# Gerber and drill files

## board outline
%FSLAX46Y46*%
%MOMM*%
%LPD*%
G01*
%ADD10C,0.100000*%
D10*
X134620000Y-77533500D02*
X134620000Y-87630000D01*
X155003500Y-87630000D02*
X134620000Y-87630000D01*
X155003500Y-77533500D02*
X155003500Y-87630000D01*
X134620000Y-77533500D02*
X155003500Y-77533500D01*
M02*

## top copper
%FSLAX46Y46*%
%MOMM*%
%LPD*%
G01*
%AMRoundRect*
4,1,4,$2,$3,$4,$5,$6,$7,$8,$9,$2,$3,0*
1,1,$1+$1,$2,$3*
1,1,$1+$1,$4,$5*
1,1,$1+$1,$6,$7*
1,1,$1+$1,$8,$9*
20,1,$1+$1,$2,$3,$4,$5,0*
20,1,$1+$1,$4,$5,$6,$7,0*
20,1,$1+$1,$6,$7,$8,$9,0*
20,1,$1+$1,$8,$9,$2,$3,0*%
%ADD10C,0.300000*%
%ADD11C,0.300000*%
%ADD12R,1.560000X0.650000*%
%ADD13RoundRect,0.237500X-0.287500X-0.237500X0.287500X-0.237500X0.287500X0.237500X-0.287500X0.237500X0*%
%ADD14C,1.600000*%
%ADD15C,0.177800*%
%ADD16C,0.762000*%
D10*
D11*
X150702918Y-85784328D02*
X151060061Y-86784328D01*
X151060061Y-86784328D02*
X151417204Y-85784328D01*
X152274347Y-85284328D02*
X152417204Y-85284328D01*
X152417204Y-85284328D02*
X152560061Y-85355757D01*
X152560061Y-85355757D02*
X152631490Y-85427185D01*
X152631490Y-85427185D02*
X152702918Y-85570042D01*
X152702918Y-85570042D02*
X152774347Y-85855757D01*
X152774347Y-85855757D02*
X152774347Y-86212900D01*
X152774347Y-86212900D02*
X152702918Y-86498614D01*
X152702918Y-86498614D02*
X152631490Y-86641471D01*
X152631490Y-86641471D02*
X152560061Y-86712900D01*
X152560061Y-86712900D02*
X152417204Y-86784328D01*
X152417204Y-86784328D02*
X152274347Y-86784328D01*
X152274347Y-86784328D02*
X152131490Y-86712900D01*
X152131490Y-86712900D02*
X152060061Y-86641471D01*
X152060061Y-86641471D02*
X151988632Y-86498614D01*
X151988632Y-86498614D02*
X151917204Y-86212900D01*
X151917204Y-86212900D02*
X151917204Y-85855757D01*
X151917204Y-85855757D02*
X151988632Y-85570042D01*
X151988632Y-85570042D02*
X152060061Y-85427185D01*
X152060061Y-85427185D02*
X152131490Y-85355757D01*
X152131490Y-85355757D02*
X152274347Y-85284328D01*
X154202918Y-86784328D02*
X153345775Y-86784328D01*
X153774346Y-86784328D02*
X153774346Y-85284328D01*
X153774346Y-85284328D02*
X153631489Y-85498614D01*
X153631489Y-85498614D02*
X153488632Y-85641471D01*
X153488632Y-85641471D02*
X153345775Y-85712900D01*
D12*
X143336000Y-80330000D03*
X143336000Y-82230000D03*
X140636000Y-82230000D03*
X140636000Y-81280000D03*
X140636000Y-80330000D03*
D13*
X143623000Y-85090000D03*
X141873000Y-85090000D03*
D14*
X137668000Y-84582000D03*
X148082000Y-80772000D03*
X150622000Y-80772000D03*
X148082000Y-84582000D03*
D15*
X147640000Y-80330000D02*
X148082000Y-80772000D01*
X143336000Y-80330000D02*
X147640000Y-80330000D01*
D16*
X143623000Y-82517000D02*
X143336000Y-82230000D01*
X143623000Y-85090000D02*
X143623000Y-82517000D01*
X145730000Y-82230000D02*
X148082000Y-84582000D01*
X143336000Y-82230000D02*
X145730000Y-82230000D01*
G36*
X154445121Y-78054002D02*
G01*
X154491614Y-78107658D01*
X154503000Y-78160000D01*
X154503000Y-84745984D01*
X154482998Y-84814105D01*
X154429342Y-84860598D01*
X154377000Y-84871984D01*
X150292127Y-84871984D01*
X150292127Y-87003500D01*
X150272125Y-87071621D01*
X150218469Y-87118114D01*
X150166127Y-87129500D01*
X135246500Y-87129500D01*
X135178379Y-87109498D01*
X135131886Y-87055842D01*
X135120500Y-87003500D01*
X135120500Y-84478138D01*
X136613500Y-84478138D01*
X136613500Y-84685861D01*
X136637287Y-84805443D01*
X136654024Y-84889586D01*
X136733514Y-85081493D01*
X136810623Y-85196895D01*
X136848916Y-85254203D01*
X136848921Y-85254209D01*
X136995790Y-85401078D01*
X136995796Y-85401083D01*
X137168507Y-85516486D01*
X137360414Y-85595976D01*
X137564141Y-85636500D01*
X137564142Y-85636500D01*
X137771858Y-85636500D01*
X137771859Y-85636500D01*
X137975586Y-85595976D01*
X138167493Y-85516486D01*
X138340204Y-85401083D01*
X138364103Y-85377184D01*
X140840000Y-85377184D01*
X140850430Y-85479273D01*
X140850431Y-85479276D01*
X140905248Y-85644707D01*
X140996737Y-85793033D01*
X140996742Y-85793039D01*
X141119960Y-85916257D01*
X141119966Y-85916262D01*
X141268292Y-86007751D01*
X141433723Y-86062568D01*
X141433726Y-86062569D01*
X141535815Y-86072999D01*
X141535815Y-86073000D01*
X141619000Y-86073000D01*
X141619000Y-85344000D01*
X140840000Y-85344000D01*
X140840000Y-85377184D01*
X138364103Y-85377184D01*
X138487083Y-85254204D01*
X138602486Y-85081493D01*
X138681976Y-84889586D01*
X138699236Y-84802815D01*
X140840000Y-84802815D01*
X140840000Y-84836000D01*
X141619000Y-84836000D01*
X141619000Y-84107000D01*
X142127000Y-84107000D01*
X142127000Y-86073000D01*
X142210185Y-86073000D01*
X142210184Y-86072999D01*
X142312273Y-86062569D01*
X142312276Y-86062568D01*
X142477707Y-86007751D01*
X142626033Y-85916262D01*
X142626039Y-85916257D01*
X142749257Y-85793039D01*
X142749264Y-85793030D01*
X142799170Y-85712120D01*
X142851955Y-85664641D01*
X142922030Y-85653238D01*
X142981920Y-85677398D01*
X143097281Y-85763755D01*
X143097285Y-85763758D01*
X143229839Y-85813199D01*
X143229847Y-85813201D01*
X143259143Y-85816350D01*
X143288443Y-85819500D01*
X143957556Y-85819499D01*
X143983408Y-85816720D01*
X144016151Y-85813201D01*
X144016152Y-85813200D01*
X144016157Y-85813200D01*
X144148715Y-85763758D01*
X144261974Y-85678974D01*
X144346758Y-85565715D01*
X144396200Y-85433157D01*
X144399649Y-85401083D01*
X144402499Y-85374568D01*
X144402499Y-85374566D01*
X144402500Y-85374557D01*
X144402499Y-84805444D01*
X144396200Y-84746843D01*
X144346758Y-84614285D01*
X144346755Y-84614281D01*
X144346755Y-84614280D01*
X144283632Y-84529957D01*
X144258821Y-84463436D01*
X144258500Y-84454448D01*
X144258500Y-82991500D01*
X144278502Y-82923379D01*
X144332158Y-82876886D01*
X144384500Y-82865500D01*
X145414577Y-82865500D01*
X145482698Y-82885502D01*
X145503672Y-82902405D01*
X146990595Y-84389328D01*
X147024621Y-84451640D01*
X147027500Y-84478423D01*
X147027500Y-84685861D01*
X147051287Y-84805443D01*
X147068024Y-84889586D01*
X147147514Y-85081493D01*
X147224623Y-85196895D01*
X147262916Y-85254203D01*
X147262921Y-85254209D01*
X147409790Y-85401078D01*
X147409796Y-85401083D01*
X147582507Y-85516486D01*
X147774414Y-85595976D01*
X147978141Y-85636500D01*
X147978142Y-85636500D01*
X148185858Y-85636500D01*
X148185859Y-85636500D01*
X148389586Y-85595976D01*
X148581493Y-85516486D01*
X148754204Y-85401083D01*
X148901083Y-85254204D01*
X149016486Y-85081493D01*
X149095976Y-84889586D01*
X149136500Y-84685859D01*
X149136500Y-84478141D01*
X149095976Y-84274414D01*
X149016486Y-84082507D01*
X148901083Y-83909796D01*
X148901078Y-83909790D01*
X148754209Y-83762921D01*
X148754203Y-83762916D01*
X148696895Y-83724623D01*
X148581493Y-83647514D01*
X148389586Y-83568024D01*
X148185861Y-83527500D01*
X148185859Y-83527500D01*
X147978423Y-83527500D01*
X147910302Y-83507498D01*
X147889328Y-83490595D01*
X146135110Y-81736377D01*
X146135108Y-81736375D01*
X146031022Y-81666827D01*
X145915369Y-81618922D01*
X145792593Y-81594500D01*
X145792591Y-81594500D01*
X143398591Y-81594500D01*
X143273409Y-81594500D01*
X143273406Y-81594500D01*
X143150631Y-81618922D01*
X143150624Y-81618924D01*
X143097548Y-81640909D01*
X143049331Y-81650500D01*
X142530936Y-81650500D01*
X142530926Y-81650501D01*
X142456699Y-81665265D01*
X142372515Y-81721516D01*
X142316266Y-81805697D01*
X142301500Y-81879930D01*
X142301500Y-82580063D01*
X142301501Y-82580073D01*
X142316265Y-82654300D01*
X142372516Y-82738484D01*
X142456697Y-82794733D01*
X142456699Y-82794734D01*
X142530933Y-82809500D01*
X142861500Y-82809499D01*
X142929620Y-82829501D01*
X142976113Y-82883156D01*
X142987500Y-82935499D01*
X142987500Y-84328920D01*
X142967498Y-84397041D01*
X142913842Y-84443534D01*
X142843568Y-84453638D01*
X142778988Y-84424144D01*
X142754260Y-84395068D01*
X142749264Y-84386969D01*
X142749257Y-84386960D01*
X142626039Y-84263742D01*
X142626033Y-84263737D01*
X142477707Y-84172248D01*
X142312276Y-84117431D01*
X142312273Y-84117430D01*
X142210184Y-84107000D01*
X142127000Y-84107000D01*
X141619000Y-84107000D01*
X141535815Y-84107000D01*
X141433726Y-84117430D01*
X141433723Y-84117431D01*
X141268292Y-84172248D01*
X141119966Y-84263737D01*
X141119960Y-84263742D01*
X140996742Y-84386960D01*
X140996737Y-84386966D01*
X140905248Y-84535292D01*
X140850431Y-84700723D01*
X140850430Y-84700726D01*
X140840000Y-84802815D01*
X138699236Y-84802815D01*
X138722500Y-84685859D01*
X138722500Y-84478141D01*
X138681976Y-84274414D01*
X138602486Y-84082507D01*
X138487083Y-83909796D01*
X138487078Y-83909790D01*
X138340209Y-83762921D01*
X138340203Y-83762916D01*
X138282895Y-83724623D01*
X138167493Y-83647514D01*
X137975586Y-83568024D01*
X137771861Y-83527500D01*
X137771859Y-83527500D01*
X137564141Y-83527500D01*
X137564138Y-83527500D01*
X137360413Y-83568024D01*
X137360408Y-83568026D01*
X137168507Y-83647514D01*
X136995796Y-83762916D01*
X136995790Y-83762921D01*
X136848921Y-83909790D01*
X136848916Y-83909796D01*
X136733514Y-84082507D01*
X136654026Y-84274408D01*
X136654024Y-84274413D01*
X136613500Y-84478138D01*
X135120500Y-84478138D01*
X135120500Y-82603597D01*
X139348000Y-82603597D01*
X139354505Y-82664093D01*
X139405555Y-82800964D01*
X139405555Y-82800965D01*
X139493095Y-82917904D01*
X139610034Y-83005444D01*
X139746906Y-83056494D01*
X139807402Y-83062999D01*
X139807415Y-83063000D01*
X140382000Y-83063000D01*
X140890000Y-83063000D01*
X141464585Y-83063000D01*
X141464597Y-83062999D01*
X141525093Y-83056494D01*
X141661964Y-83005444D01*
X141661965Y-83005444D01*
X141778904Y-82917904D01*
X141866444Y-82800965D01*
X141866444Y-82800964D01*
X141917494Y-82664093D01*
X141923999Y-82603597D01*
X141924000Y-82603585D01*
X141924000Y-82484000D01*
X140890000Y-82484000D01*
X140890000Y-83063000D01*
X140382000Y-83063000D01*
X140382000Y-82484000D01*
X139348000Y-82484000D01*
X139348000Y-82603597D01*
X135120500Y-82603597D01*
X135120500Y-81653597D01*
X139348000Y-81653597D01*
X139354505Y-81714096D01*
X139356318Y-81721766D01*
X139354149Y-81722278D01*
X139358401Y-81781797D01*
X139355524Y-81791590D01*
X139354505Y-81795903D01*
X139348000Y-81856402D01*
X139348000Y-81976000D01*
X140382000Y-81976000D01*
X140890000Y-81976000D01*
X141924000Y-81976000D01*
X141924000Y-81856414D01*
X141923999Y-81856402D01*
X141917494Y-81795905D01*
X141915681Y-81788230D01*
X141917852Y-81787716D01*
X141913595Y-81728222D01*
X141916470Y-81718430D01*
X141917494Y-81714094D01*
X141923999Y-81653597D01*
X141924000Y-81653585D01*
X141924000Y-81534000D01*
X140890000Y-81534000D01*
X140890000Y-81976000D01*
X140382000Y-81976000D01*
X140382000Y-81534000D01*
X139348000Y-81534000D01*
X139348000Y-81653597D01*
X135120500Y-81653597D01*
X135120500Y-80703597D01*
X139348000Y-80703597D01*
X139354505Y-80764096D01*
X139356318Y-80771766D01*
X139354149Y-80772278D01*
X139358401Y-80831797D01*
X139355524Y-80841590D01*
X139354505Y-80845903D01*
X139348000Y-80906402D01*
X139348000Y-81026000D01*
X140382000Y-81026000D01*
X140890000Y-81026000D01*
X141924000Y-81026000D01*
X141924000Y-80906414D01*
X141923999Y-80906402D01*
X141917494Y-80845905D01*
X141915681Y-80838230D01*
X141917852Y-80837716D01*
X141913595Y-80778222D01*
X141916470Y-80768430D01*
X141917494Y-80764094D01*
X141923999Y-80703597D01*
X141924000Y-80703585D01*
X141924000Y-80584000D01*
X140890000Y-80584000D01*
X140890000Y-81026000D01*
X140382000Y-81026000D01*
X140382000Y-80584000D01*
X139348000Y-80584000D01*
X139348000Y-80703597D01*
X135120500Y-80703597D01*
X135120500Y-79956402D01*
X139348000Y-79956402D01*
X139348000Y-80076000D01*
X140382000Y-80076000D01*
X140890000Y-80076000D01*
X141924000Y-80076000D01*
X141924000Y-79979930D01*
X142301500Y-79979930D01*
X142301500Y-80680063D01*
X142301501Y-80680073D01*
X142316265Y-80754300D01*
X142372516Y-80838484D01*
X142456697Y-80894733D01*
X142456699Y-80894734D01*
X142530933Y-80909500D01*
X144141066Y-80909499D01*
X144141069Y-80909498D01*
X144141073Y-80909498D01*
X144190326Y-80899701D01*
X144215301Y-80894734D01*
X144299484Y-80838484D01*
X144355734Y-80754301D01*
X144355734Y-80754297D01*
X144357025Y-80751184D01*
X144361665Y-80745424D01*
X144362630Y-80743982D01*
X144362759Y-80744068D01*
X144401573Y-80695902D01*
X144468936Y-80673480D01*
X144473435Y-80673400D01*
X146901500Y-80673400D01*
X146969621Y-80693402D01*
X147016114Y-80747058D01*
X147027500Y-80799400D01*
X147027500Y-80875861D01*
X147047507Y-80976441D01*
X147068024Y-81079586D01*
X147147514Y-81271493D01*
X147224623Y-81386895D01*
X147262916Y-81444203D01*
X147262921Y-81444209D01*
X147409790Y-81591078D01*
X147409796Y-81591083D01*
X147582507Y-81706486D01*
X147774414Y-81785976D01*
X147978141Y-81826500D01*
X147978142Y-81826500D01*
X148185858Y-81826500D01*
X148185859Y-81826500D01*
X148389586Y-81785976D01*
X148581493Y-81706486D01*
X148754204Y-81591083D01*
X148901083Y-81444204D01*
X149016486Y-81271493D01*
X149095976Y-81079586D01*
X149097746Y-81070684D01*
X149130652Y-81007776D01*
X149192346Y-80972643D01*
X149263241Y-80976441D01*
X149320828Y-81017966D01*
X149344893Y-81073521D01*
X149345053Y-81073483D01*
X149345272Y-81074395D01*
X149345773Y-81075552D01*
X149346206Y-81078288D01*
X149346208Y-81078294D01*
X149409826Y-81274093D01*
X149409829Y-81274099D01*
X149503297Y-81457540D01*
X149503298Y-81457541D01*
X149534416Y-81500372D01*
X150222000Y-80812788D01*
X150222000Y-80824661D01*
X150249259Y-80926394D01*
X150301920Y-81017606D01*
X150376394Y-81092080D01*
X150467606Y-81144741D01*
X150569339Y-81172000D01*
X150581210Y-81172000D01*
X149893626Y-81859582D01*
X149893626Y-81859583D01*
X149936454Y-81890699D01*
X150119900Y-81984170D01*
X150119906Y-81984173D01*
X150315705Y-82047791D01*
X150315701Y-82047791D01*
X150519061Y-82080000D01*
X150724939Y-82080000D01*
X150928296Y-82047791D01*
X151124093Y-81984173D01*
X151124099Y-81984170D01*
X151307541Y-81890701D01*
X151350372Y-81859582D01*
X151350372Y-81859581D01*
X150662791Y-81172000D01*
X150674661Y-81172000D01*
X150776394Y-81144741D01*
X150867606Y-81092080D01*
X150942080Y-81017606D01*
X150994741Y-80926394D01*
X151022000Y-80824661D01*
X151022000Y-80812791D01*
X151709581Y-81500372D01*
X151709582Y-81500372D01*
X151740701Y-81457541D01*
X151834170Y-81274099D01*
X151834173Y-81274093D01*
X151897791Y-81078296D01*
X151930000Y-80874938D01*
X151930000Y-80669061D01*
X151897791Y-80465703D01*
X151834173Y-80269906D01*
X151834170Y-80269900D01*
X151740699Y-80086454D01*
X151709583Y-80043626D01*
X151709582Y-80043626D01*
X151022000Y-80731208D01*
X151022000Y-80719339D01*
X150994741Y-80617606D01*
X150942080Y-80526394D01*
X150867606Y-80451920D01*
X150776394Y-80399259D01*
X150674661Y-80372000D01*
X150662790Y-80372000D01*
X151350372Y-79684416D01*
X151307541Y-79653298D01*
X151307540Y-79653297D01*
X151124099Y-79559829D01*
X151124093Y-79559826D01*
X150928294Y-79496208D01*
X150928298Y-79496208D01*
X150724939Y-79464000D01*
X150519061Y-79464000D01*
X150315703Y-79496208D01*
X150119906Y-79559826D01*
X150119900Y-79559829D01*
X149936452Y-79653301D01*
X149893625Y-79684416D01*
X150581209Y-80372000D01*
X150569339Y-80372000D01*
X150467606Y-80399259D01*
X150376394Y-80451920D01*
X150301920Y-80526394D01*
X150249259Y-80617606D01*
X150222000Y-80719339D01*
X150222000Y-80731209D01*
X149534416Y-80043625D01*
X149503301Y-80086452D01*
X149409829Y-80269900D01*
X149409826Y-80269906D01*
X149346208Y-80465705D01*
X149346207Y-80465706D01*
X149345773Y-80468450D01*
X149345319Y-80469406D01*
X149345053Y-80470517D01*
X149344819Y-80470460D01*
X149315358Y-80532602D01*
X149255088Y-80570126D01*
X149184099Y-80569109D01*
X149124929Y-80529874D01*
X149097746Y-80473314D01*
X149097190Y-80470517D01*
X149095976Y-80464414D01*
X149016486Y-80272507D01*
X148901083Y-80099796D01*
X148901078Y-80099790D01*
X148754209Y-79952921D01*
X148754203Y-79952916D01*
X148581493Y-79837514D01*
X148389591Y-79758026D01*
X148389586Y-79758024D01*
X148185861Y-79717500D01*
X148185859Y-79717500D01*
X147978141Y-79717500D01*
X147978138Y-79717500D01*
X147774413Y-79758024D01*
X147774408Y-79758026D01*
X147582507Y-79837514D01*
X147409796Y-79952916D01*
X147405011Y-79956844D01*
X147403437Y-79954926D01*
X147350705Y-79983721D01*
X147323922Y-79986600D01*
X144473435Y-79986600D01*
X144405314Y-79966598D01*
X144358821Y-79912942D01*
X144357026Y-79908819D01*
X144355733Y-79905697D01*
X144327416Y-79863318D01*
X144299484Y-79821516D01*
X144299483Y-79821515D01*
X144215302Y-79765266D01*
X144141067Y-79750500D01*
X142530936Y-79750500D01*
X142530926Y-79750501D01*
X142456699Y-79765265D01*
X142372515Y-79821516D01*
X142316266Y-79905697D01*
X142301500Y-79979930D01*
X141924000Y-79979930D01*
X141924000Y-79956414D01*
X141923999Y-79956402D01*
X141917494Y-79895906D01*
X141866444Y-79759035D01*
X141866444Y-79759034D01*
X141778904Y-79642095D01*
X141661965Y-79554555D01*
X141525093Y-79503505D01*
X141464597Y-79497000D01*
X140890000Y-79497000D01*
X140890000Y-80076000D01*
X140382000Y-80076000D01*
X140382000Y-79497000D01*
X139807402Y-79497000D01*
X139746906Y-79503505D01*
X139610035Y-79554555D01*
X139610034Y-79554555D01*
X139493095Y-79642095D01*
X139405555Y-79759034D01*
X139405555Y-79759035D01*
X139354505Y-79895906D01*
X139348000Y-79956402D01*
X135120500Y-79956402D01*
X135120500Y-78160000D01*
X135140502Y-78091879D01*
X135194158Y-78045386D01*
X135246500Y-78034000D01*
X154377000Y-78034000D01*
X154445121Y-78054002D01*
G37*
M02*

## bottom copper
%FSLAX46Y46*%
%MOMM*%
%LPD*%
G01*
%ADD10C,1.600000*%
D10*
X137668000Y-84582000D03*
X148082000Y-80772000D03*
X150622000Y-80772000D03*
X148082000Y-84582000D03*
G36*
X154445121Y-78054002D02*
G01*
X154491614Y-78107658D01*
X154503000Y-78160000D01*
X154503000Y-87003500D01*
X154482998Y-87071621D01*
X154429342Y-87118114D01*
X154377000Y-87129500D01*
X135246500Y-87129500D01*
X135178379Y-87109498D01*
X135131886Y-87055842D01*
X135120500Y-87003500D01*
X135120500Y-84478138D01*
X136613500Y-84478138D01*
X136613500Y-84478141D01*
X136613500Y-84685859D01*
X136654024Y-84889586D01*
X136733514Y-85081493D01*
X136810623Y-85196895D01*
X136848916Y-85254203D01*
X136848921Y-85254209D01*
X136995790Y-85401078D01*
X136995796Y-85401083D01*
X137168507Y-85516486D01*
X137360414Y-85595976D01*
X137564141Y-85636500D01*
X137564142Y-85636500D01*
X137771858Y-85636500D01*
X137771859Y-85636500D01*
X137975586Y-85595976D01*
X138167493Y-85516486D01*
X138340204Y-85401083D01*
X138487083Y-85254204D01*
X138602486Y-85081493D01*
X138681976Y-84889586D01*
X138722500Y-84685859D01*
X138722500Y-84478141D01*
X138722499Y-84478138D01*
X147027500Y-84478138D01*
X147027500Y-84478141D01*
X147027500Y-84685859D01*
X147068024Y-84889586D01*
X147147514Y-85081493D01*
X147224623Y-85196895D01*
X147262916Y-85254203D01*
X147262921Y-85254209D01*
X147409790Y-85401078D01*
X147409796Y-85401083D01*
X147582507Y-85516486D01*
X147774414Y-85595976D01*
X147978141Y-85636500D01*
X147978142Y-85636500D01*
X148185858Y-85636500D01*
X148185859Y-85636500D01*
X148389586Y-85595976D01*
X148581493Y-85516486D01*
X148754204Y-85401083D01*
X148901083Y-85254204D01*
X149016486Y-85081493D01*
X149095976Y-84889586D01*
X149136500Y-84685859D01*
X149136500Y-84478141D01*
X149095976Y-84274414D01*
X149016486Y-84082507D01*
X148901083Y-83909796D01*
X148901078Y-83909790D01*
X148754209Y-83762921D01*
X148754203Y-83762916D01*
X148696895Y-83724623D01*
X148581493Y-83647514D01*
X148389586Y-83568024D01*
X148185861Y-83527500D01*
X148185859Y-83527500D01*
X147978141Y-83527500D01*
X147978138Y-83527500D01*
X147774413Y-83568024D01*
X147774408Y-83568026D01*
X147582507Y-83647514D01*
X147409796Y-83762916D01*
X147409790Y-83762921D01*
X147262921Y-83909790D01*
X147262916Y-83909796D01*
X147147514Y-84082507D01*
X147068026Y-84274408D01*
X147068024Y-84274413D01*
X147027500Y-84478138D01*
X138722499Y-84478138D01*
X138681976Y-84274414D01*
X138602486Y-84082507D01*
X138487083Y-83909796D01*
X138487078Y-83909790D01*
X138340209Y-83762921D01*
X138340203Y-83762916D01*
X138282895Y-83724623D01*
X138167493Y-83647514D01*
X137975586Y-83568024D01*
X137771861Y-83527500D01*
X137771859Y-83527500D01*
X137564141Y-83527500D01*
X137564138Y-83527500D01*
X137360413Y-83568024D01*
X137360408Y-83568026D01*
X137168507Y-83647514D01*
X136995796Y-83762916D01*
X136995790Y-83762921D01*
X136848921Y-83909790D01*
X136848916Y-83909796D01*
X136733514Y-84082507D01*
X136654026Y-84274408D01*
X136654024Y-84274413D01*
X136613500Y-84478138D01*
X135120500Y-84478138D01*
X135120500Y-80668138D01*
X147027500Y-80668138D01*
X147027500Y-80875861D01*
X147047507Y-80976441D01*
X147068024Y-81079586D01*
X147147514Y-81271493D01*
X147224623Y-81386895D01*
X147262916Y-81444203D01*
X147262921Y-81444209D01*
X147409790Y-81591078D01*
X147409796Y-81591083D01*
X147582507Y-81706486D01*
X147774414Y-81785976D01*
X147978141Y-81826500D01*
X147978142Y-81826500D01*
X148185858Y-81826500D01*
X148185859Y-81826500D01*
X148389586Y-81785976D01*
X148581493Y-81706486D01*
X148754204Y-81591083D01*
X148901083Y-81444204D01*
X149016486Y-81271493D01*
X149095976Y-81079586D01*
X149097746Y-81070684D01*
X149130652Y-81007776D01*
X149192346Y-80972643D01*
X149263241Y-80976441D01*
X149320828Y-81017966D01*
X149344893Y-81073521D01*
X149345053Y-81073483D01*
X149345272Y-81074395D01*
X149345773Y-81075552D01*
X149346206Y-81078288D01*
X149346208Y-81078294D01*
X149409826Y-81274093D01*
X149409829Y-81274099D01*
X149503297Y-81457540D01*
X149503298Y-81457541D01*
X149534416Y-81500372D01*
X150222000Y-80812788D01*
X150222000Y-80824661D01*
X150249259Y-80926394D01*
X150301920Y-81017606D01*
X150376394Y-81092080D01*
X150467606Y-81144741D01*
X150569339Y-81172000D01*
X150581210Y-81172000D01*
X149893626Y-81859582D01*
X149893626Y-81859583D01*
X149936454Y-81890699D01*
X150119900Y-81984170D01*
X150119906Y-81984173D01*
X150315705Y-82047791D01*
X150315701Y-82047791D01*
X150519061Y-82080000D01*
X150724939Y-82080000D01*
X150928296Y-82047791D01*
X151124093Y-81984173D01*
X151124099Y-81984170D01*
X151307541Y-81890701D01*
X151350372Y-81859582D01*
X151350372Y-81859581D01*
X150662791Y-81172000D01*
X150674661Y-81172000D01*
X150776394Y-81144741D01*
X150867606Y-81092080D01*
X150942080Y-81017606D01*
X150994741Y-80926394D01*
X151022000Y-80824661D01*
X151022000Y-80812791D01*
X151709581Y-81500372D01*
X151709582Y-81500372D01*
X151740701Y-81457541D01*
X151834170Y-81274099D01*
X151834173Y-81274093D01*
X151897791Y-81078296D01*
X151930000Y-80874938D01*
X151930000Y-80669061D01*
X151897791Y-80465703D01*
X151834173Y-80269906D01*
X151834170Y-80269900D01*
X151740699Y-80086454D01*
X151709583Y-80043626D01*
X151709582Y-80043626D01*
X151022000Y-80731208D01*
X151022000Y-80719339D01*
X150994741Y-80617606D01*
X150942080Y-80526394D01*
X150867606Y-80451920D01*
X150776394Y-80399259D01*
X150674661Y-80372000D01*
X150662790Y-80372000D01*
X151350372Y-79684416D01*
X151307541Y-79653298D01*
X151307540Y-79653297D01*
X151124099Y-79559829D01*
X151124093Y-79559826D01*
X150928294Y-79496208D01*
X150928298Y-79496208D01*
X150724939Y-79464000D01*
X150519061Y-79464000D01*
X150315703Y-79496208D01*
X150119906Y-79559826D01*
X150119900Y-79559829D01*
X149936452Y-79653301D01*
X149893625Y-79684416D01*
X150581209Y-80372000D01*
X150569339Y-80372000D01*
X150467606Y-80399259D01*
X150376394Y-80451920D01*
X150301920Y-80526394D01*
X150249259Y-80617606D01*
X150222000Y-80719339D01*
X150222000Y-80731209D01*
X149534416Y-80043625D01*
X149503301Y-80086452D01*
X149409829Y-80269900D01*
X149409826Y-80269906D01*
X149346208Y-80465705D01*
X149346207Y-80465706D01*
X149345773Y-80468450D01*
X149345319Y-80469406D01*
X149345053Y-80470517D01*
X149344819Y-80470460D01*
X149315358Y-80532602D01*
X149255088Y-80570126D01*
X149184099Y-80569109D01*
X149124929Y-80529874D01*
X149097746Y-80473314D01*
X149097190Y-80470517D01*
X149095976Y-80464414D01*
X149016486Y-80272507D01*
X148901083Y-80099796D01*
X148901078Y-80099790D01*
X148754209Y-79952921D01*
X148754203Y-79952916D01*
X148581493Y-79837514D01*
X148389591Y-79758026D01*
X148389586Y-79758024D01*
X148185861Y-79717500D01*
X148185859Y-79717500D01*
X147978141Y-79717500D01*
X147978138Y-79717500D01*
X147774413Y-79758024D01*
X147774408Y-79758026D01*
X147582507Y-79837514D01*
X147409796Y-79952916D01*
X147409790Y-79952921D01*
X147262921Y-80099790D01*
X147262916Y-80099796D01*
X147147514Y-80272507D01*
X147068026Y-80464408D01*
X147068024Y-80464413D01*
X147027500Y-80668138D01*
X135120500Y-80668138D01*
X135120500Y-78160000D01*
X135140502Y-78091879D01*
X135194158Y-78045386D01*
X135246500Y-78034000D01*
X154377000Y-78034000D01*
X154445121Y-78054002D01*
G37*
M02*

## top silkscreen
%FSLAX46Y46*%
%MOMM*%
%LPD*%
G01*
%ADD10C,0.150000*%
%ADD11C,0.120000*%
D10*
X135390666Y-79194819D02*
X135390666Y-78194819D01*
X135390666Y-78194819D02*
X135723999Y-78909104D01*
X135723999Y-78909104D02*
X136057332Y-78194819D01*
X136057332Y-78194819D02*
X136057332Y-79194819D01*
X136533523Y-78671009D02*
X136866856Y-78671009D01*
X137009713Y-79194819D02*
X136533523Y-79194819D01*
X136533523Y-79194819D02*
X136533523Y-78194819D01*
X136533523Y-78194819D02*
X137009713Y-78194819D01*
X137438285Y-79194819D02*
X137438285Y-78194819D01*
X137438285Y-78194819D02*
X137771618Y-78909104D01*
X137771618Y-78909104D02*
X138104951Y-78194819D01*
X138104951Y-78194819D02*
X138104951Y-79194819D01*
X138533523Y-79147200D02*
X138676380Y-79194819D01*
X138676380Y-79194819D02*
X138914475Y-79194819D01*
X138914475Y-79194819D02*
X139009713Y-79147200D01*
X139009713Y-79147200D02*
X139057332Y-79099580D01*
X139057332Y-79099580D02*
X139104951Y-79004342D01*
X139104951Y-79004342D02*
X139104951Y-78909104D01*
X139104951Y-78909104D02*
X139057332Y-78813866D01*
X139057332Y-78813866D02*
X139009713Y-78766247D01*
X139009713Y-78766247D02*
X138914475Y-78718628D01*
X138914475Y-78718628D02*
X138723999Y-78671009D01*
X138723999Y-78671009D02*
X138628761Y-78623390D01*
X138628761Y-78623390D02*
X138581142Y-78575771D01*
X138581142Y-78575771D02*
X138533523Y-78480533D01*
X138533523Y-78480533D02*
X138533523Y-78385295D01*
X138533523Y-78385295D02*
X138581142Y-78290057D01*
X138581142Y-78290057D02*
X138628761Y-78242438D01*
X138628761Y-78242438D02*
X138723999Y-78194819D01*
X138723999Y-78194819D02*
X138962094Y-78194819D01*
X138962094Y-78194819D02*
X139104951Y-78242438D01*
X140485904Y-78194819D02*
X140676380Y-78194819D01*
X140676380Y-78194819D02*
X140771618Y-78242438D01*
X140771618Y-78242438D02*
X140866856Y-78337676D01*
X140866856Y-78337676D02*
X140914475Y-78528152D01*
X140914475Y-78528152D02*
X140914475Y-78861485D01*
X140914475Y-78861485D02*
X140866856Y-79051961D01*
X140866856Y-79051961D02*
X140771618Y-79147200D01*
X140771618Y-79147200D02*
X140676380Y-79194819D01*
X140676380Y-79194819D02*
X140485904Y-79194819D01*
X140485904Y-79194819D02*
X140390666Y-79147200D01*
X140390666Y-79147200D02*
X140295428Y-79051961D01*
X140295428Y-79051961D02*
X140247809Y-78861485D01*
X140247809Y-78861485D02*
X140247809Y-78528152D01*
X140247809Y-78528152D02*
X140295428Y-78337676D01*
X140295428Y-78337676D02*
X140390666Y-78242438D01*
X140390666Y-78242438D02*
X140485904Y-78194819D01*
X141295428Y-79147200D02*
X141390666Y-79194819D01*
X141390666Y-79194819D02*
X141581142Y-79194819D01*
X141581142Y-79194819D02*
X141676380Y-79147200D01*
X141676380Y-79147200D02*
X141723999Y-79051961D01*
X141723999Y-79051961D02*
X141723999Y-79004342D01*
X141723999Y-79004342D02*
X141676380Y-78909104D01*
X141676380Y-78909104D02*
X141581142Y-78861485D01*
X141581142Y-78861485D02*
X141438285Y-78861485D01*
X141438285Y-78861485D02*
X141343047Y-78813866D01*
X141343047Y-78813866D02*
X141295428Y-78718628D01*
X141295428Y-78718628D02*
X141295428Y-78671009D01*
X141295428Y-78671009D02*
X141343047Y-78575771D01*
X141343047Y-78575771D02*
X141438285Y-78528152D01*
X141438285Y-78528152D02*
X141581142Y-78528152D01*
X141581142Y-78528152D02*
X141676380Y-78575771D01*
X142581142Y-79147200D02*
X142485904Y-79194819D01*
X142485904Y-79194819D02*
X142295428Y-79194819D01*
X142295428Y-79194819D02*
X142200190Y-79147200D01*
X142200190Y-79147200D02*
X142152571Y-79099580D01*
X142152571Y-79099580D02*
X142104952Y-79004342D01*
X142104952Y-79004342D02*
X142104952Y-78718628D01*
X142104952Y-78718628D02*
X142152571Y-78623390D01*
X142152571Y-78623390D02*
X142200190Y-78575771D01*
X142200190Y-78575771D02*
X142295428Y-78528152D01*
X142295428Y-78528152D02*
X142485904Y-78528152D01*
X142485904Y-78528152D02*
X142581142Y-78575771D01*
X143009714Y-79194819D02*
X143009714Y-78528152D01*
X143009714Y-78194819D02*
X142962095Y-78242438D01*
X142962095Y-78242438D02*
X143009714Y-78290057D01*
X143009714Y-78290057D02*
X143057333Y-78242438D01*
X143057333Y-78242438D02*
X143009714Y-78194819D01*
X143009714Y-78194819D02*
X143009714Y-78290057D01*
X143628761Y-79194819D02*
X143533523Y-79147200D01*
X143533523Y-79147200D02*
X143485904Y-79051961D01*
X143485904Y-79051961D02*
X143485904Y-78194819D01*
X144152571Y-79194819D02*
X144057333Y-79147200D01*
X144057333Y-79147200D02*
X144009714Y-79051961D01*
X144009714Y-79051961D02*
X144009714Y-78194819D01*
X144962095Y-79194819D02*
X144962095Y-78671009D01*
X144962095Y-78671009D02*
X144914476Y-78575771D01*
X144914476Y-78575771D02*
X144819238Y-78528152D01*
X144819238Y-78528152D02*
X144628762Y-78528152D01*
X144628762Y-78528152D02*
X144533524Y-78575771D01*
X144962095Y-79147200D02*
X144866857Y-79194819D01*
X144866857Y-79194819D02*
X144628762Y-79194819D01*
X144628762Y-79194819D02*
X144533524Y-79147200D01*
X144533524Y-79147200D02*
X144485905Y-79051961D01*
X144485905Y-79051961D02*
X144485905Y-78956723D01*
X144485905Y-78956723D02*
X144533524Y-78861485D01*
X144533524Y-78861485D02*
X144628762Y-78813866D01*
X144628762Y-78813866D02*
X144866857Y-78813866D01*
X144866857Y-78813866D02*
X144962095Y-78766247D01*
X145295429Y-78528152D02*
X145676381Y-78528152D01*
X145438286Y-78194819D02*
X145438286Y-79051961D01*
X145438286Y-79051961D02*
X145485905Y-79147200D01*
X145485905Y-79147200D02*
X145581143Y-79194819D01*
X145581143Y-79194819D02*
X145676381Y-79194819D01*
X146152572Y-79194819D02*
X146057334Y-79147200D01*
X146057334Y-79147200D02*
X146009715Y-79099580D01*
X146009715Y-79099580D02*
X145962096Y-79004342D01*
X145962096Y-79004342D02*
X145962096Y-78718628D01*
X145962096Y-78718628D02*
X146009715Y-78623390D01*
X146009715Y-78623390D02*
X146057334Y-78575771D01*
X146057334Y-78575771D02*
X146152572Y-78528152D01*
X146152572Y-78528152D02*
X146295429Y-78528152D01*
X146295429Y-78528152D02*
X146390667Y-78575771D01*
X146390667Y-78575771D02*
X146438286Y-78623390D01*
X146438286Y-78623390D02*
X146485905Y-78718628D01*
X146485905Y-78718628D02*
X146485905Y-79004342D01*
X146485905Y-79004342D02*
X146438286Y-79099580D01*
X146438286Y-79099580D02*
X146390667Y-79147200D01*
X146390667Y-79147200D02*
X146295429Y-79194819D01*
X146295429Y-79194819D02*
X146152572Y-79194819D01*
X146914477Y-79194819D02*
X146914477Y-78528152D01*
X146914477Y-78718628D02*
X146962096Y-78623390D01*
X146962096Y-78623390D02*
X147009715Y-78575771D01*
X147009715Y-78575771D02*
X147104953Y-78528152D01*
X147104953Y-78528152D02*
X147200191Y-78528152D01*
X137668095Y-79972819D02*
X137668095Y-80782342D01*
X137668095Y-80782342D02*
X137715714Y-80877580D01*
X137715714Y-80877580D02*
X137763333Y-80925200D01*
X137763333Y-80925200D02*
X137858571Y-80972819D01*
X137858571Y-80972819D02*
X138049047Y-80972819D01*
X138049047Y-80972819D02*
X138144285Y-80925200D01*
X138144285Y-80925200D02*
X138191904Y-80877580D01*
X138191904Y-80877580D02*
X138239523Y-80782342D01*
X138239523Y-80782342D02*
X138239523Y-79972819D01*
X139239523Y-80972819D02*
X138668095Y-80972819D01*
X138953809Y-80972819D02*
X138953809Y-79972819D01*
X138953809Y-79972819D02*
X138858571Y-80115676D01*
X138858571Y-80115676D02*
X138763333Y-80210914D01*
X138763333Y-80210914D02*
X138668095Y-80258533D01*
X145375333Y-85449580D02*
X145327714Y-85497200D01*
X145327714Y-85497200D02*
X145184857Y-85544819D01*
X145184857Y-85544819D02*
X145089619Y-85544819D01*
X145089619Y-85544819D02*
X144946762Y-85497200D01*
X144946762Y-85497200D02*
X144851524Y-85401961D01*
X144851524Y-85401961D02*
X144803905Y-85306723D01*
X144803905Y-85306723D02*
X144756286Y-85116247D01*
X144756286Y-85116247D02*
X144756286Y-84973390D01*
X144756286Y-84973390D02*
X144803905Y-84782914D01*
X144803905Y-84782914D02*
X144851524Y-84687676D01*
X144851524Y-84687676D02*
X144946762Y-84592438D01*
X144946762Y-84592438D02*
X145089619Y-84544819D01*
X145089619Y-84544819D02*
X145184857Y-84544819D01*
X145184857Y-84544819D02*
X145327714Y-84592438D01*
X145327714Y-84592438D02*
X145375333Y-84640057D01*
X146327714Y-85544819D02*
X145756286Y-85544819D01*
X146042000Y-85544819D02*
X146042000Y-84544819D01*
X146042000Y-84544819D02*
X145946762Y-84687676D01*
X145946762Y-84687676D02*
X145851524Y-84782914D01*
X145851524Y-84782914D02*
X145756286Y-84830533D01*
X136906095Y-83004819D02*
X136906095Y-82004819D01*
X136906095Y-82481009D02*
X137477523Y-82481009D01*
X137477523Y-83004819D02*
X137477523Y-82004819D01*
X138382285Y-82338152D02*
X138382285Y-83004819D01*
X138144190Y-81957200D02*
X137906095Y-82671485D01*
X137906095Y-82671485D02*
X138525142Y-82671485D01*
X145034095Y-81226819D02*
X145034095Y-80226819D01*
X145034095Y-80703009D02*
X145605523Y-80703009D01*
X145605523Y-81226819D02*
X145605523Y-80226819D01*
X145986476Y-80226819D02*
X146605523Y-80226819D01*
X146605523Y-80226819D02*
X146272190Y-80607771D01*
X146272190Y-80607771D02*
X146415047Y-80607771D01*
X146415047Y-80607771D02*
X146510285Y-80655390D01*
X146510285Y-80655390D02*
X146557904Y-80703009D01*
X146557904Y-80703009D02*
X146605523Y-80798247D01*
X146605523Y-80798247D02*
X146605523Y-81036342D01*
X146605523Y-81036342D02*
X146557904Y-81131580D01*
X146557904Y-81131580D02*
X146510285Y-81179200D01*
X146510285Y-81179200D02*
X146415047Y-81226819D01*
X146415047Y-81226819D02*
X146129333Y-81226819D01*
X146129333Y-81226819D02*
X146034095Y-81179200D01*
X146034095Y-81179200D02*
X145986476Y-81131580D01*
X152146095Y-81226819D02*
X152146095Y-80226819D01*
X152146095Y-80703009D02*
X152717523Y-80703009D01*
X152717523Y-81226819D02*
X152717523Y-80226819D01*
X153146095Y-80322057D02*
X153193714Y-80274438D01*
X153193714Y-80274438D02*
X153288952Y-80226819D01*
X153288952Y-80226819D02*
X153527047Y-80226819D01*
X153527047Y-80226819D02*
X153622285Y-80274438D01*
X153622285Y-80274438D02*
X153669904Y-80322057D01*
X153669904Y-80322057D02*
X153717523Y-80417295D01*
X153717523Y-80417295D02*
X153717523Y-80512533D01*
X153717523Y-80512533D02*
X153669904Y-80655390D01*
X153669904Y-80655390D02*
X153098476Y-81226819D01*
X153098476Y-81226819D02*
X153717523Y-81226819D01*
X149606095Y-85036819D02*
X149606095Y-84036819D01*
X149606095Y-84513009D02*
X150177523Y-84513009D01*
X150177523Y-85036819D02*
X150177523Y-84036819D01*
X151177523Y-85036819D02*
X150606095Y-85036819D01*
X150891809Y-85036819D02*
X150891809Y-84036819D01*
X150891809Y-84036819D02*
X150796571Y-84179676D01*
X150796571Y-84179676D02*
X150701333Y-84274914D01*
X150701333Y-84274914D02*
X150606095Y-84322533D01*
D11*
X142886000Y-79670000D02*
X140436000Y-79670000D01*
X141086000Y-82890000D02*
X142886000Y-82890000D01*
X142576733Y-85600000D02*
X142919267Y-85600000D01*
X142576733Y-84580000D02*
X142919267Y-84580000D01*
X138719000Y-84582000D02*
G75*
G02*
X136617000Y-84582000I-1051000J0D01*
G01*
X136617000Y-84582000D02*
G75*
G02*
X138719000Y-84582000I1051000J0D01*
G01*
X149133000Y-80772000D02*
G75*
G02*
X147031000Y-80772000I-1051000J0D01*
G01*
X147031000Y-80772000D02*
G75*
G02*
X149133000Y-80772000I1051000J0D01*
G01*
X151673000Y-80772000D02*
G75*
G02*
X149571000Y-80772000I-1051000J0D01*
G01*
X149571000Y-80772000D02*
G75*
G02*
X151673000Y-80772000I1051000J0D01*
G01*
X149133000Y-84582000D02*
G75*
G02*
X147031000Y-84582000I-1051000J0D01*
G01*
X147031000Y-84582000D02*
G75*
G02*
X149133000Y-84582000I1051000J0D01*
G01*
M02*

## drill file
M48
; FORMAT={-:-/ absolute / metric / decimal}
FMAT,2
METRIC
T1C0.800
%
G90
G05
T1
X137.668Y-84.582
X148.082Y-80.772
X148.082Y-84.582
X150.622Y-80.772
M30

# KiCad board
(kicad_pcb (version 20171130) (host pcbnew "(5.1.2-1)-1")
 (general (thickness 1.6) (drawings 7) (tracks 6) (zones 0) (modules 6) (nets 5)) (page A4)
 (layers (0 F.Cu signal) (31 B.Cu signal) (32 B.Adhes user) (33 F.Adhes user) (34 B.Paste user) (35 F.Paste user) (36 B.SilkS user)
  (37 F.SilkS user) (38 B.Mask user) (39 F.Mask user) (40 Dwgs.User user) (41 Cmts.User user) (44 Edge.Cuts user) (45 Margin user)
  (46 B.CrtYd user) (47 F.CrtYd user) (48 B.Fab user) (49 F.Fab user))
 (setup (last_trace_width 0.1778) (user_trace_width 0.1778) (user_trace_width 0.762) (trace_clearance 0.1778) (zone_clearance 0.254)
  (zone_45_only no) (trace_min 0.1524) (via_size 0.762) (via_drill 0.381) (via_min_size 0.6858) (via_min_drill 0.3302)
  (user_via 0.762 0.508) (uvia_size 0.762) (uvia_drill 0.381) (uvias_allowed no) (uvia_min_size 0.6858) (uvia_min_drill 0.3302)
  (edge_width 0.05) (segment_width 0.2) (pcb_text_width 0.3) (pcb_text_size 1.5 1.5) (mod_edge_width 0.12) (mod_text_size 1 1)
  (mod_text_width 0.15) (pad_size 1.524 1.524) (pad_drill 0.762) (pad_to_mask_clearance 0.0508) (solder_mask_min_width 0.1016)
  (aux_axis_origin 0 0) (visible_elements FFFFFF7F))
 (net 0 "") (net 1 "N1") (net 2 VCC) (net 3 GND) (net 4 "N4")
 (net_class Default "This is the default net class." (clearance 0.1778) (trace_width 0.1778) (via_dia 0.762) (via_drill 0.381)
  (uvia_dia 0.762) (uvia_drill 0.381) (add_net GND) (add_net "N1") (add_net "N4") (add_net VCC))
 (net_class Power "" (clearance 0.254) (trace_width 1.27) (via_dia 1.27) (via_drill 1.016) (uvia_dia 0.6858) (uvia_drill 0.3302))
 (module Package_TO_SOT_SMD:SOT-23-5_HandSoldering (layer F.Cu) (at 141.986 81.28)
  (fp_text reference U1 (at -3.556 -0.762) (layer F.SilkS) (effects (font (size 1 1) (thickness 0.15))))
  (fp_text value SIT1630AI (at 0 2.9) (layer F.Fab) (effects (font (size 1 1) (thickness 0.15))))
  (fp_line (start 0.9 -1.61) (end -1.55 -1.61) (layer F.SilkS) (width 0.12))
  (fp_line (start -0.9 1.61) (end 0.9 1.61) (layer F.SilkS) (width 0.12))
  (pad 5 smd rect (at 1.35 -0.95) (size 1.56 0.65) (layers F.Cu F.Paste F.Mask) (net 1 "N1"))
  (pad 4 smd rect (at 1.35 0.95) (size 1.56 0.65) (layers F.Cu F.Paste F.Mask) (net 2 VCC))
  (pad 3 smd rect (at -1.35 0.95) (size 1.56 0.65) (layers F.Cu F.Paste F.Mask) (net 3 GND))
  (pad 2 smd rect (at -1.35 0) (size 1.56 0.65) (layers F.Cu F.Paste F.Mask) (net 3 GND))
  (pad 1 smd rect (at -1.35 -0.95) (size 1.56 0.65) (layers F.Cu F.Paste F.Mask) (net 3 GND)))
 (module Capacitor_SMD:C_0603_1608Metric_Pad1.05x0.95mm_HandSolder (layer F.Cu) (at 142.748 85.09)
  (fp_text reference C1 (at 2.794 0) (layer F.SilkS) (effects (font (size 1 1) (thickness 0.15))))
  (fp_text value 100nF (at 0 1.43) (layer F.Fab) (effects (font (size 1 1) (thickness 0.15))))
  (fp_line (start -0.171267 0.51) (end 0.171267 0.51) (layer F.SilkS) (width 0.12))
  (fp_line (start -0.171267 -0.51) (end 0.171267 -0.51) (layer F.SilkS) (width 0.12))
  (pad 2 smd roundrect (at 0.875 0) (size 1.05 0.95) (layers F.Cu F.Paste F.Mask) (roundrect_rratio 0.25) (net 2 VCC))
  (pad 1 smd roundrect (at -0.875 0) (size 1.05 0.95) (layers F.Cu F.Paste F.Mask) (roundrect_rratio 0.25) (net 3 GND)))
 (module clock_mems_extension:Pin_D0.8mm (layer F.Cu) (at 137.668 84.582)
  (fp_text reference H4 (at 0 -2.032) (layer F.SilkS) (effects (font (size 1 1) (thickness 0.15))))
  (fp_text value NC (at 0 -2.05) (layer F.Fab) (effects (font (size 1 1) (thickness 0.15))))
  (fp_circle (center 0 0) (end 1.051 0) (layer F.SilkS) (width 0.12))
  (pad 1 thru_hole circle (at 0 0) (size 1.6 1.6) (drill 0.8) (layers *.Cu *.Mask) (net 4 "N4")))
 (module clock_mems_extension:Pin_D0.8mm (layer F.Cu) (at 148.082 80.772)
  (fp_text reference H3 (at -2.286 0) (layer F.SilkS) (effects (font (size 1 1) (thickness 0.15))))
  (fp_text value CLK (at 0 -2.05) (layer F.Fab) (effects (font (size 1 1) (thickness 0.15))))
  (fp_circle (center 0 0) (end 1.051 0) (layer F.SilkS) (width 0.12))
  (pad 1 thru_hole circle (at 0 0) (size 1.6 1.6) (drill 0.8) (layers *.Cu *.Mask) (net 1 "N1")))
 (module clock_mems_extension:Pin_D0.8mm (layer F.Cu) (at 150.622 80.772)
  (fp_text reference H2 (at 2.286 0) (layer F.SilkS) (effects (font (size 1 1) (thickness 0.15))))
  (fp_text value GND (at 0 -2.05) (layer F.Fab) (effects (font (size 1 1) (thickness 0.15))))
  (fp_circle (center 0 0) (end 1.051 0) (layer F.SilkS) (width 0.12))
  (pad 1 thru_hole circle (at 0 0) (size 1.6 1.6) (drill 0.8) (layers *.Cu *.Mask) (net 3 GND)))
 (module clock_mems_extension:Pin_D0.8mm (layer F.Cu) (at 148.082 84.582)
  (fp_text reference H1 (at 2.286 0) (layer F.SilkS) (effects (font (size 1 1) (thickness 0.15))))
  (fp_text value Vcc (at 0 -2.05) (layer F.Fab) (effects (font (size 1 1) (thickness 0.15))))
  (fp_circle (center 0 0) (end 1.051 0) (layer F.SilkS) (width 0.12))
  (pad 1 thru_hole circle (at 0 0) (size 1.6 1.6) (drill 0.8) (layers *.Cu *.Mask) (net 2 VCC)))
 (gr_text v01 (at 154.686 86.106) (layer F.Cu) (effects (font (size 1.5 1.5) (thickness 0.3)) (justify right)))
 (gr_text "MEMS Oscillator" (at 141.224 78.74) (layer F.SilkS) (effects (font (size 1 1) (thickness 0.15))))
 (gr_line (start 134.62 77.5335) (end 134.62 87.63) (layer Edge.Cuts) (width 0.1))
 (gr_line (start 155.0035 87.63) (end 134.62 87.63) (layer Edge.Cuts) (width 0.1))
 (gr_line (start 155.0035 77.5335) (end 155.0035 87.63) (layer Edge.Cuts) (width 0.1))
 (gr_line (start 134.62 77.5335) (end 155.0035 77.5335) (layer Edge.Cuts) (width 0.1))
 (segment (start 147.64 80.33) (end 148.082 80.772) (width 0.1778) (layer F.Cu) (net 1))
 (segment (start 143.336 80.33) (end 147.64 80.33) (width 0.1778) (layer F.Cu) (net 1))
 (segment (start 143.623 82.517) (end 143.336 82.23) (width 0.762) (layer F.Cu) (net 2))
 (segment (start 143.623 85.09) (end 143.623 82.517) (width 0.762) (layer F.Cu) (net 2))
 (segment (start 145.73 82.23) (end 148.082 84.582) (width 0.762) (layer F.Cu) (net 2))
 (segment (start 143.336 82.23) (end 145.73 82.23) (width 0.762) (layer F.Cu) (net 2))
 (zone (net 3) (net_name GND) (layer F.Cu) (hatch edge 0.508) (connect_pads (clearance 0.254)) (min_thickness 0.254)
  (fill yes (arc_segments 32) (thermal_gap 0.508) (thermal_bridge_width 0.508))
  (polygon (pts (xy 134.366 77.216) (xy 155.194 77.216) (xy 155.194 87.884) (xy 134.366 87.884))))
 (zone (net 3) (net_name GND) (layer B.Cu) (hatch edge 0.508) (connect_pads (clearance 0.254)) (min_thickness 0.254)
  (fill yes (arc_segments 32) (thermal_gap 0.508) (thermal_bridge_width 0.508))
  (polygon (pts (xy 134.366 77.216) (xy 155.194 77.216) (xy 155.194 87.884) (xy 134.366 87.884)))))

